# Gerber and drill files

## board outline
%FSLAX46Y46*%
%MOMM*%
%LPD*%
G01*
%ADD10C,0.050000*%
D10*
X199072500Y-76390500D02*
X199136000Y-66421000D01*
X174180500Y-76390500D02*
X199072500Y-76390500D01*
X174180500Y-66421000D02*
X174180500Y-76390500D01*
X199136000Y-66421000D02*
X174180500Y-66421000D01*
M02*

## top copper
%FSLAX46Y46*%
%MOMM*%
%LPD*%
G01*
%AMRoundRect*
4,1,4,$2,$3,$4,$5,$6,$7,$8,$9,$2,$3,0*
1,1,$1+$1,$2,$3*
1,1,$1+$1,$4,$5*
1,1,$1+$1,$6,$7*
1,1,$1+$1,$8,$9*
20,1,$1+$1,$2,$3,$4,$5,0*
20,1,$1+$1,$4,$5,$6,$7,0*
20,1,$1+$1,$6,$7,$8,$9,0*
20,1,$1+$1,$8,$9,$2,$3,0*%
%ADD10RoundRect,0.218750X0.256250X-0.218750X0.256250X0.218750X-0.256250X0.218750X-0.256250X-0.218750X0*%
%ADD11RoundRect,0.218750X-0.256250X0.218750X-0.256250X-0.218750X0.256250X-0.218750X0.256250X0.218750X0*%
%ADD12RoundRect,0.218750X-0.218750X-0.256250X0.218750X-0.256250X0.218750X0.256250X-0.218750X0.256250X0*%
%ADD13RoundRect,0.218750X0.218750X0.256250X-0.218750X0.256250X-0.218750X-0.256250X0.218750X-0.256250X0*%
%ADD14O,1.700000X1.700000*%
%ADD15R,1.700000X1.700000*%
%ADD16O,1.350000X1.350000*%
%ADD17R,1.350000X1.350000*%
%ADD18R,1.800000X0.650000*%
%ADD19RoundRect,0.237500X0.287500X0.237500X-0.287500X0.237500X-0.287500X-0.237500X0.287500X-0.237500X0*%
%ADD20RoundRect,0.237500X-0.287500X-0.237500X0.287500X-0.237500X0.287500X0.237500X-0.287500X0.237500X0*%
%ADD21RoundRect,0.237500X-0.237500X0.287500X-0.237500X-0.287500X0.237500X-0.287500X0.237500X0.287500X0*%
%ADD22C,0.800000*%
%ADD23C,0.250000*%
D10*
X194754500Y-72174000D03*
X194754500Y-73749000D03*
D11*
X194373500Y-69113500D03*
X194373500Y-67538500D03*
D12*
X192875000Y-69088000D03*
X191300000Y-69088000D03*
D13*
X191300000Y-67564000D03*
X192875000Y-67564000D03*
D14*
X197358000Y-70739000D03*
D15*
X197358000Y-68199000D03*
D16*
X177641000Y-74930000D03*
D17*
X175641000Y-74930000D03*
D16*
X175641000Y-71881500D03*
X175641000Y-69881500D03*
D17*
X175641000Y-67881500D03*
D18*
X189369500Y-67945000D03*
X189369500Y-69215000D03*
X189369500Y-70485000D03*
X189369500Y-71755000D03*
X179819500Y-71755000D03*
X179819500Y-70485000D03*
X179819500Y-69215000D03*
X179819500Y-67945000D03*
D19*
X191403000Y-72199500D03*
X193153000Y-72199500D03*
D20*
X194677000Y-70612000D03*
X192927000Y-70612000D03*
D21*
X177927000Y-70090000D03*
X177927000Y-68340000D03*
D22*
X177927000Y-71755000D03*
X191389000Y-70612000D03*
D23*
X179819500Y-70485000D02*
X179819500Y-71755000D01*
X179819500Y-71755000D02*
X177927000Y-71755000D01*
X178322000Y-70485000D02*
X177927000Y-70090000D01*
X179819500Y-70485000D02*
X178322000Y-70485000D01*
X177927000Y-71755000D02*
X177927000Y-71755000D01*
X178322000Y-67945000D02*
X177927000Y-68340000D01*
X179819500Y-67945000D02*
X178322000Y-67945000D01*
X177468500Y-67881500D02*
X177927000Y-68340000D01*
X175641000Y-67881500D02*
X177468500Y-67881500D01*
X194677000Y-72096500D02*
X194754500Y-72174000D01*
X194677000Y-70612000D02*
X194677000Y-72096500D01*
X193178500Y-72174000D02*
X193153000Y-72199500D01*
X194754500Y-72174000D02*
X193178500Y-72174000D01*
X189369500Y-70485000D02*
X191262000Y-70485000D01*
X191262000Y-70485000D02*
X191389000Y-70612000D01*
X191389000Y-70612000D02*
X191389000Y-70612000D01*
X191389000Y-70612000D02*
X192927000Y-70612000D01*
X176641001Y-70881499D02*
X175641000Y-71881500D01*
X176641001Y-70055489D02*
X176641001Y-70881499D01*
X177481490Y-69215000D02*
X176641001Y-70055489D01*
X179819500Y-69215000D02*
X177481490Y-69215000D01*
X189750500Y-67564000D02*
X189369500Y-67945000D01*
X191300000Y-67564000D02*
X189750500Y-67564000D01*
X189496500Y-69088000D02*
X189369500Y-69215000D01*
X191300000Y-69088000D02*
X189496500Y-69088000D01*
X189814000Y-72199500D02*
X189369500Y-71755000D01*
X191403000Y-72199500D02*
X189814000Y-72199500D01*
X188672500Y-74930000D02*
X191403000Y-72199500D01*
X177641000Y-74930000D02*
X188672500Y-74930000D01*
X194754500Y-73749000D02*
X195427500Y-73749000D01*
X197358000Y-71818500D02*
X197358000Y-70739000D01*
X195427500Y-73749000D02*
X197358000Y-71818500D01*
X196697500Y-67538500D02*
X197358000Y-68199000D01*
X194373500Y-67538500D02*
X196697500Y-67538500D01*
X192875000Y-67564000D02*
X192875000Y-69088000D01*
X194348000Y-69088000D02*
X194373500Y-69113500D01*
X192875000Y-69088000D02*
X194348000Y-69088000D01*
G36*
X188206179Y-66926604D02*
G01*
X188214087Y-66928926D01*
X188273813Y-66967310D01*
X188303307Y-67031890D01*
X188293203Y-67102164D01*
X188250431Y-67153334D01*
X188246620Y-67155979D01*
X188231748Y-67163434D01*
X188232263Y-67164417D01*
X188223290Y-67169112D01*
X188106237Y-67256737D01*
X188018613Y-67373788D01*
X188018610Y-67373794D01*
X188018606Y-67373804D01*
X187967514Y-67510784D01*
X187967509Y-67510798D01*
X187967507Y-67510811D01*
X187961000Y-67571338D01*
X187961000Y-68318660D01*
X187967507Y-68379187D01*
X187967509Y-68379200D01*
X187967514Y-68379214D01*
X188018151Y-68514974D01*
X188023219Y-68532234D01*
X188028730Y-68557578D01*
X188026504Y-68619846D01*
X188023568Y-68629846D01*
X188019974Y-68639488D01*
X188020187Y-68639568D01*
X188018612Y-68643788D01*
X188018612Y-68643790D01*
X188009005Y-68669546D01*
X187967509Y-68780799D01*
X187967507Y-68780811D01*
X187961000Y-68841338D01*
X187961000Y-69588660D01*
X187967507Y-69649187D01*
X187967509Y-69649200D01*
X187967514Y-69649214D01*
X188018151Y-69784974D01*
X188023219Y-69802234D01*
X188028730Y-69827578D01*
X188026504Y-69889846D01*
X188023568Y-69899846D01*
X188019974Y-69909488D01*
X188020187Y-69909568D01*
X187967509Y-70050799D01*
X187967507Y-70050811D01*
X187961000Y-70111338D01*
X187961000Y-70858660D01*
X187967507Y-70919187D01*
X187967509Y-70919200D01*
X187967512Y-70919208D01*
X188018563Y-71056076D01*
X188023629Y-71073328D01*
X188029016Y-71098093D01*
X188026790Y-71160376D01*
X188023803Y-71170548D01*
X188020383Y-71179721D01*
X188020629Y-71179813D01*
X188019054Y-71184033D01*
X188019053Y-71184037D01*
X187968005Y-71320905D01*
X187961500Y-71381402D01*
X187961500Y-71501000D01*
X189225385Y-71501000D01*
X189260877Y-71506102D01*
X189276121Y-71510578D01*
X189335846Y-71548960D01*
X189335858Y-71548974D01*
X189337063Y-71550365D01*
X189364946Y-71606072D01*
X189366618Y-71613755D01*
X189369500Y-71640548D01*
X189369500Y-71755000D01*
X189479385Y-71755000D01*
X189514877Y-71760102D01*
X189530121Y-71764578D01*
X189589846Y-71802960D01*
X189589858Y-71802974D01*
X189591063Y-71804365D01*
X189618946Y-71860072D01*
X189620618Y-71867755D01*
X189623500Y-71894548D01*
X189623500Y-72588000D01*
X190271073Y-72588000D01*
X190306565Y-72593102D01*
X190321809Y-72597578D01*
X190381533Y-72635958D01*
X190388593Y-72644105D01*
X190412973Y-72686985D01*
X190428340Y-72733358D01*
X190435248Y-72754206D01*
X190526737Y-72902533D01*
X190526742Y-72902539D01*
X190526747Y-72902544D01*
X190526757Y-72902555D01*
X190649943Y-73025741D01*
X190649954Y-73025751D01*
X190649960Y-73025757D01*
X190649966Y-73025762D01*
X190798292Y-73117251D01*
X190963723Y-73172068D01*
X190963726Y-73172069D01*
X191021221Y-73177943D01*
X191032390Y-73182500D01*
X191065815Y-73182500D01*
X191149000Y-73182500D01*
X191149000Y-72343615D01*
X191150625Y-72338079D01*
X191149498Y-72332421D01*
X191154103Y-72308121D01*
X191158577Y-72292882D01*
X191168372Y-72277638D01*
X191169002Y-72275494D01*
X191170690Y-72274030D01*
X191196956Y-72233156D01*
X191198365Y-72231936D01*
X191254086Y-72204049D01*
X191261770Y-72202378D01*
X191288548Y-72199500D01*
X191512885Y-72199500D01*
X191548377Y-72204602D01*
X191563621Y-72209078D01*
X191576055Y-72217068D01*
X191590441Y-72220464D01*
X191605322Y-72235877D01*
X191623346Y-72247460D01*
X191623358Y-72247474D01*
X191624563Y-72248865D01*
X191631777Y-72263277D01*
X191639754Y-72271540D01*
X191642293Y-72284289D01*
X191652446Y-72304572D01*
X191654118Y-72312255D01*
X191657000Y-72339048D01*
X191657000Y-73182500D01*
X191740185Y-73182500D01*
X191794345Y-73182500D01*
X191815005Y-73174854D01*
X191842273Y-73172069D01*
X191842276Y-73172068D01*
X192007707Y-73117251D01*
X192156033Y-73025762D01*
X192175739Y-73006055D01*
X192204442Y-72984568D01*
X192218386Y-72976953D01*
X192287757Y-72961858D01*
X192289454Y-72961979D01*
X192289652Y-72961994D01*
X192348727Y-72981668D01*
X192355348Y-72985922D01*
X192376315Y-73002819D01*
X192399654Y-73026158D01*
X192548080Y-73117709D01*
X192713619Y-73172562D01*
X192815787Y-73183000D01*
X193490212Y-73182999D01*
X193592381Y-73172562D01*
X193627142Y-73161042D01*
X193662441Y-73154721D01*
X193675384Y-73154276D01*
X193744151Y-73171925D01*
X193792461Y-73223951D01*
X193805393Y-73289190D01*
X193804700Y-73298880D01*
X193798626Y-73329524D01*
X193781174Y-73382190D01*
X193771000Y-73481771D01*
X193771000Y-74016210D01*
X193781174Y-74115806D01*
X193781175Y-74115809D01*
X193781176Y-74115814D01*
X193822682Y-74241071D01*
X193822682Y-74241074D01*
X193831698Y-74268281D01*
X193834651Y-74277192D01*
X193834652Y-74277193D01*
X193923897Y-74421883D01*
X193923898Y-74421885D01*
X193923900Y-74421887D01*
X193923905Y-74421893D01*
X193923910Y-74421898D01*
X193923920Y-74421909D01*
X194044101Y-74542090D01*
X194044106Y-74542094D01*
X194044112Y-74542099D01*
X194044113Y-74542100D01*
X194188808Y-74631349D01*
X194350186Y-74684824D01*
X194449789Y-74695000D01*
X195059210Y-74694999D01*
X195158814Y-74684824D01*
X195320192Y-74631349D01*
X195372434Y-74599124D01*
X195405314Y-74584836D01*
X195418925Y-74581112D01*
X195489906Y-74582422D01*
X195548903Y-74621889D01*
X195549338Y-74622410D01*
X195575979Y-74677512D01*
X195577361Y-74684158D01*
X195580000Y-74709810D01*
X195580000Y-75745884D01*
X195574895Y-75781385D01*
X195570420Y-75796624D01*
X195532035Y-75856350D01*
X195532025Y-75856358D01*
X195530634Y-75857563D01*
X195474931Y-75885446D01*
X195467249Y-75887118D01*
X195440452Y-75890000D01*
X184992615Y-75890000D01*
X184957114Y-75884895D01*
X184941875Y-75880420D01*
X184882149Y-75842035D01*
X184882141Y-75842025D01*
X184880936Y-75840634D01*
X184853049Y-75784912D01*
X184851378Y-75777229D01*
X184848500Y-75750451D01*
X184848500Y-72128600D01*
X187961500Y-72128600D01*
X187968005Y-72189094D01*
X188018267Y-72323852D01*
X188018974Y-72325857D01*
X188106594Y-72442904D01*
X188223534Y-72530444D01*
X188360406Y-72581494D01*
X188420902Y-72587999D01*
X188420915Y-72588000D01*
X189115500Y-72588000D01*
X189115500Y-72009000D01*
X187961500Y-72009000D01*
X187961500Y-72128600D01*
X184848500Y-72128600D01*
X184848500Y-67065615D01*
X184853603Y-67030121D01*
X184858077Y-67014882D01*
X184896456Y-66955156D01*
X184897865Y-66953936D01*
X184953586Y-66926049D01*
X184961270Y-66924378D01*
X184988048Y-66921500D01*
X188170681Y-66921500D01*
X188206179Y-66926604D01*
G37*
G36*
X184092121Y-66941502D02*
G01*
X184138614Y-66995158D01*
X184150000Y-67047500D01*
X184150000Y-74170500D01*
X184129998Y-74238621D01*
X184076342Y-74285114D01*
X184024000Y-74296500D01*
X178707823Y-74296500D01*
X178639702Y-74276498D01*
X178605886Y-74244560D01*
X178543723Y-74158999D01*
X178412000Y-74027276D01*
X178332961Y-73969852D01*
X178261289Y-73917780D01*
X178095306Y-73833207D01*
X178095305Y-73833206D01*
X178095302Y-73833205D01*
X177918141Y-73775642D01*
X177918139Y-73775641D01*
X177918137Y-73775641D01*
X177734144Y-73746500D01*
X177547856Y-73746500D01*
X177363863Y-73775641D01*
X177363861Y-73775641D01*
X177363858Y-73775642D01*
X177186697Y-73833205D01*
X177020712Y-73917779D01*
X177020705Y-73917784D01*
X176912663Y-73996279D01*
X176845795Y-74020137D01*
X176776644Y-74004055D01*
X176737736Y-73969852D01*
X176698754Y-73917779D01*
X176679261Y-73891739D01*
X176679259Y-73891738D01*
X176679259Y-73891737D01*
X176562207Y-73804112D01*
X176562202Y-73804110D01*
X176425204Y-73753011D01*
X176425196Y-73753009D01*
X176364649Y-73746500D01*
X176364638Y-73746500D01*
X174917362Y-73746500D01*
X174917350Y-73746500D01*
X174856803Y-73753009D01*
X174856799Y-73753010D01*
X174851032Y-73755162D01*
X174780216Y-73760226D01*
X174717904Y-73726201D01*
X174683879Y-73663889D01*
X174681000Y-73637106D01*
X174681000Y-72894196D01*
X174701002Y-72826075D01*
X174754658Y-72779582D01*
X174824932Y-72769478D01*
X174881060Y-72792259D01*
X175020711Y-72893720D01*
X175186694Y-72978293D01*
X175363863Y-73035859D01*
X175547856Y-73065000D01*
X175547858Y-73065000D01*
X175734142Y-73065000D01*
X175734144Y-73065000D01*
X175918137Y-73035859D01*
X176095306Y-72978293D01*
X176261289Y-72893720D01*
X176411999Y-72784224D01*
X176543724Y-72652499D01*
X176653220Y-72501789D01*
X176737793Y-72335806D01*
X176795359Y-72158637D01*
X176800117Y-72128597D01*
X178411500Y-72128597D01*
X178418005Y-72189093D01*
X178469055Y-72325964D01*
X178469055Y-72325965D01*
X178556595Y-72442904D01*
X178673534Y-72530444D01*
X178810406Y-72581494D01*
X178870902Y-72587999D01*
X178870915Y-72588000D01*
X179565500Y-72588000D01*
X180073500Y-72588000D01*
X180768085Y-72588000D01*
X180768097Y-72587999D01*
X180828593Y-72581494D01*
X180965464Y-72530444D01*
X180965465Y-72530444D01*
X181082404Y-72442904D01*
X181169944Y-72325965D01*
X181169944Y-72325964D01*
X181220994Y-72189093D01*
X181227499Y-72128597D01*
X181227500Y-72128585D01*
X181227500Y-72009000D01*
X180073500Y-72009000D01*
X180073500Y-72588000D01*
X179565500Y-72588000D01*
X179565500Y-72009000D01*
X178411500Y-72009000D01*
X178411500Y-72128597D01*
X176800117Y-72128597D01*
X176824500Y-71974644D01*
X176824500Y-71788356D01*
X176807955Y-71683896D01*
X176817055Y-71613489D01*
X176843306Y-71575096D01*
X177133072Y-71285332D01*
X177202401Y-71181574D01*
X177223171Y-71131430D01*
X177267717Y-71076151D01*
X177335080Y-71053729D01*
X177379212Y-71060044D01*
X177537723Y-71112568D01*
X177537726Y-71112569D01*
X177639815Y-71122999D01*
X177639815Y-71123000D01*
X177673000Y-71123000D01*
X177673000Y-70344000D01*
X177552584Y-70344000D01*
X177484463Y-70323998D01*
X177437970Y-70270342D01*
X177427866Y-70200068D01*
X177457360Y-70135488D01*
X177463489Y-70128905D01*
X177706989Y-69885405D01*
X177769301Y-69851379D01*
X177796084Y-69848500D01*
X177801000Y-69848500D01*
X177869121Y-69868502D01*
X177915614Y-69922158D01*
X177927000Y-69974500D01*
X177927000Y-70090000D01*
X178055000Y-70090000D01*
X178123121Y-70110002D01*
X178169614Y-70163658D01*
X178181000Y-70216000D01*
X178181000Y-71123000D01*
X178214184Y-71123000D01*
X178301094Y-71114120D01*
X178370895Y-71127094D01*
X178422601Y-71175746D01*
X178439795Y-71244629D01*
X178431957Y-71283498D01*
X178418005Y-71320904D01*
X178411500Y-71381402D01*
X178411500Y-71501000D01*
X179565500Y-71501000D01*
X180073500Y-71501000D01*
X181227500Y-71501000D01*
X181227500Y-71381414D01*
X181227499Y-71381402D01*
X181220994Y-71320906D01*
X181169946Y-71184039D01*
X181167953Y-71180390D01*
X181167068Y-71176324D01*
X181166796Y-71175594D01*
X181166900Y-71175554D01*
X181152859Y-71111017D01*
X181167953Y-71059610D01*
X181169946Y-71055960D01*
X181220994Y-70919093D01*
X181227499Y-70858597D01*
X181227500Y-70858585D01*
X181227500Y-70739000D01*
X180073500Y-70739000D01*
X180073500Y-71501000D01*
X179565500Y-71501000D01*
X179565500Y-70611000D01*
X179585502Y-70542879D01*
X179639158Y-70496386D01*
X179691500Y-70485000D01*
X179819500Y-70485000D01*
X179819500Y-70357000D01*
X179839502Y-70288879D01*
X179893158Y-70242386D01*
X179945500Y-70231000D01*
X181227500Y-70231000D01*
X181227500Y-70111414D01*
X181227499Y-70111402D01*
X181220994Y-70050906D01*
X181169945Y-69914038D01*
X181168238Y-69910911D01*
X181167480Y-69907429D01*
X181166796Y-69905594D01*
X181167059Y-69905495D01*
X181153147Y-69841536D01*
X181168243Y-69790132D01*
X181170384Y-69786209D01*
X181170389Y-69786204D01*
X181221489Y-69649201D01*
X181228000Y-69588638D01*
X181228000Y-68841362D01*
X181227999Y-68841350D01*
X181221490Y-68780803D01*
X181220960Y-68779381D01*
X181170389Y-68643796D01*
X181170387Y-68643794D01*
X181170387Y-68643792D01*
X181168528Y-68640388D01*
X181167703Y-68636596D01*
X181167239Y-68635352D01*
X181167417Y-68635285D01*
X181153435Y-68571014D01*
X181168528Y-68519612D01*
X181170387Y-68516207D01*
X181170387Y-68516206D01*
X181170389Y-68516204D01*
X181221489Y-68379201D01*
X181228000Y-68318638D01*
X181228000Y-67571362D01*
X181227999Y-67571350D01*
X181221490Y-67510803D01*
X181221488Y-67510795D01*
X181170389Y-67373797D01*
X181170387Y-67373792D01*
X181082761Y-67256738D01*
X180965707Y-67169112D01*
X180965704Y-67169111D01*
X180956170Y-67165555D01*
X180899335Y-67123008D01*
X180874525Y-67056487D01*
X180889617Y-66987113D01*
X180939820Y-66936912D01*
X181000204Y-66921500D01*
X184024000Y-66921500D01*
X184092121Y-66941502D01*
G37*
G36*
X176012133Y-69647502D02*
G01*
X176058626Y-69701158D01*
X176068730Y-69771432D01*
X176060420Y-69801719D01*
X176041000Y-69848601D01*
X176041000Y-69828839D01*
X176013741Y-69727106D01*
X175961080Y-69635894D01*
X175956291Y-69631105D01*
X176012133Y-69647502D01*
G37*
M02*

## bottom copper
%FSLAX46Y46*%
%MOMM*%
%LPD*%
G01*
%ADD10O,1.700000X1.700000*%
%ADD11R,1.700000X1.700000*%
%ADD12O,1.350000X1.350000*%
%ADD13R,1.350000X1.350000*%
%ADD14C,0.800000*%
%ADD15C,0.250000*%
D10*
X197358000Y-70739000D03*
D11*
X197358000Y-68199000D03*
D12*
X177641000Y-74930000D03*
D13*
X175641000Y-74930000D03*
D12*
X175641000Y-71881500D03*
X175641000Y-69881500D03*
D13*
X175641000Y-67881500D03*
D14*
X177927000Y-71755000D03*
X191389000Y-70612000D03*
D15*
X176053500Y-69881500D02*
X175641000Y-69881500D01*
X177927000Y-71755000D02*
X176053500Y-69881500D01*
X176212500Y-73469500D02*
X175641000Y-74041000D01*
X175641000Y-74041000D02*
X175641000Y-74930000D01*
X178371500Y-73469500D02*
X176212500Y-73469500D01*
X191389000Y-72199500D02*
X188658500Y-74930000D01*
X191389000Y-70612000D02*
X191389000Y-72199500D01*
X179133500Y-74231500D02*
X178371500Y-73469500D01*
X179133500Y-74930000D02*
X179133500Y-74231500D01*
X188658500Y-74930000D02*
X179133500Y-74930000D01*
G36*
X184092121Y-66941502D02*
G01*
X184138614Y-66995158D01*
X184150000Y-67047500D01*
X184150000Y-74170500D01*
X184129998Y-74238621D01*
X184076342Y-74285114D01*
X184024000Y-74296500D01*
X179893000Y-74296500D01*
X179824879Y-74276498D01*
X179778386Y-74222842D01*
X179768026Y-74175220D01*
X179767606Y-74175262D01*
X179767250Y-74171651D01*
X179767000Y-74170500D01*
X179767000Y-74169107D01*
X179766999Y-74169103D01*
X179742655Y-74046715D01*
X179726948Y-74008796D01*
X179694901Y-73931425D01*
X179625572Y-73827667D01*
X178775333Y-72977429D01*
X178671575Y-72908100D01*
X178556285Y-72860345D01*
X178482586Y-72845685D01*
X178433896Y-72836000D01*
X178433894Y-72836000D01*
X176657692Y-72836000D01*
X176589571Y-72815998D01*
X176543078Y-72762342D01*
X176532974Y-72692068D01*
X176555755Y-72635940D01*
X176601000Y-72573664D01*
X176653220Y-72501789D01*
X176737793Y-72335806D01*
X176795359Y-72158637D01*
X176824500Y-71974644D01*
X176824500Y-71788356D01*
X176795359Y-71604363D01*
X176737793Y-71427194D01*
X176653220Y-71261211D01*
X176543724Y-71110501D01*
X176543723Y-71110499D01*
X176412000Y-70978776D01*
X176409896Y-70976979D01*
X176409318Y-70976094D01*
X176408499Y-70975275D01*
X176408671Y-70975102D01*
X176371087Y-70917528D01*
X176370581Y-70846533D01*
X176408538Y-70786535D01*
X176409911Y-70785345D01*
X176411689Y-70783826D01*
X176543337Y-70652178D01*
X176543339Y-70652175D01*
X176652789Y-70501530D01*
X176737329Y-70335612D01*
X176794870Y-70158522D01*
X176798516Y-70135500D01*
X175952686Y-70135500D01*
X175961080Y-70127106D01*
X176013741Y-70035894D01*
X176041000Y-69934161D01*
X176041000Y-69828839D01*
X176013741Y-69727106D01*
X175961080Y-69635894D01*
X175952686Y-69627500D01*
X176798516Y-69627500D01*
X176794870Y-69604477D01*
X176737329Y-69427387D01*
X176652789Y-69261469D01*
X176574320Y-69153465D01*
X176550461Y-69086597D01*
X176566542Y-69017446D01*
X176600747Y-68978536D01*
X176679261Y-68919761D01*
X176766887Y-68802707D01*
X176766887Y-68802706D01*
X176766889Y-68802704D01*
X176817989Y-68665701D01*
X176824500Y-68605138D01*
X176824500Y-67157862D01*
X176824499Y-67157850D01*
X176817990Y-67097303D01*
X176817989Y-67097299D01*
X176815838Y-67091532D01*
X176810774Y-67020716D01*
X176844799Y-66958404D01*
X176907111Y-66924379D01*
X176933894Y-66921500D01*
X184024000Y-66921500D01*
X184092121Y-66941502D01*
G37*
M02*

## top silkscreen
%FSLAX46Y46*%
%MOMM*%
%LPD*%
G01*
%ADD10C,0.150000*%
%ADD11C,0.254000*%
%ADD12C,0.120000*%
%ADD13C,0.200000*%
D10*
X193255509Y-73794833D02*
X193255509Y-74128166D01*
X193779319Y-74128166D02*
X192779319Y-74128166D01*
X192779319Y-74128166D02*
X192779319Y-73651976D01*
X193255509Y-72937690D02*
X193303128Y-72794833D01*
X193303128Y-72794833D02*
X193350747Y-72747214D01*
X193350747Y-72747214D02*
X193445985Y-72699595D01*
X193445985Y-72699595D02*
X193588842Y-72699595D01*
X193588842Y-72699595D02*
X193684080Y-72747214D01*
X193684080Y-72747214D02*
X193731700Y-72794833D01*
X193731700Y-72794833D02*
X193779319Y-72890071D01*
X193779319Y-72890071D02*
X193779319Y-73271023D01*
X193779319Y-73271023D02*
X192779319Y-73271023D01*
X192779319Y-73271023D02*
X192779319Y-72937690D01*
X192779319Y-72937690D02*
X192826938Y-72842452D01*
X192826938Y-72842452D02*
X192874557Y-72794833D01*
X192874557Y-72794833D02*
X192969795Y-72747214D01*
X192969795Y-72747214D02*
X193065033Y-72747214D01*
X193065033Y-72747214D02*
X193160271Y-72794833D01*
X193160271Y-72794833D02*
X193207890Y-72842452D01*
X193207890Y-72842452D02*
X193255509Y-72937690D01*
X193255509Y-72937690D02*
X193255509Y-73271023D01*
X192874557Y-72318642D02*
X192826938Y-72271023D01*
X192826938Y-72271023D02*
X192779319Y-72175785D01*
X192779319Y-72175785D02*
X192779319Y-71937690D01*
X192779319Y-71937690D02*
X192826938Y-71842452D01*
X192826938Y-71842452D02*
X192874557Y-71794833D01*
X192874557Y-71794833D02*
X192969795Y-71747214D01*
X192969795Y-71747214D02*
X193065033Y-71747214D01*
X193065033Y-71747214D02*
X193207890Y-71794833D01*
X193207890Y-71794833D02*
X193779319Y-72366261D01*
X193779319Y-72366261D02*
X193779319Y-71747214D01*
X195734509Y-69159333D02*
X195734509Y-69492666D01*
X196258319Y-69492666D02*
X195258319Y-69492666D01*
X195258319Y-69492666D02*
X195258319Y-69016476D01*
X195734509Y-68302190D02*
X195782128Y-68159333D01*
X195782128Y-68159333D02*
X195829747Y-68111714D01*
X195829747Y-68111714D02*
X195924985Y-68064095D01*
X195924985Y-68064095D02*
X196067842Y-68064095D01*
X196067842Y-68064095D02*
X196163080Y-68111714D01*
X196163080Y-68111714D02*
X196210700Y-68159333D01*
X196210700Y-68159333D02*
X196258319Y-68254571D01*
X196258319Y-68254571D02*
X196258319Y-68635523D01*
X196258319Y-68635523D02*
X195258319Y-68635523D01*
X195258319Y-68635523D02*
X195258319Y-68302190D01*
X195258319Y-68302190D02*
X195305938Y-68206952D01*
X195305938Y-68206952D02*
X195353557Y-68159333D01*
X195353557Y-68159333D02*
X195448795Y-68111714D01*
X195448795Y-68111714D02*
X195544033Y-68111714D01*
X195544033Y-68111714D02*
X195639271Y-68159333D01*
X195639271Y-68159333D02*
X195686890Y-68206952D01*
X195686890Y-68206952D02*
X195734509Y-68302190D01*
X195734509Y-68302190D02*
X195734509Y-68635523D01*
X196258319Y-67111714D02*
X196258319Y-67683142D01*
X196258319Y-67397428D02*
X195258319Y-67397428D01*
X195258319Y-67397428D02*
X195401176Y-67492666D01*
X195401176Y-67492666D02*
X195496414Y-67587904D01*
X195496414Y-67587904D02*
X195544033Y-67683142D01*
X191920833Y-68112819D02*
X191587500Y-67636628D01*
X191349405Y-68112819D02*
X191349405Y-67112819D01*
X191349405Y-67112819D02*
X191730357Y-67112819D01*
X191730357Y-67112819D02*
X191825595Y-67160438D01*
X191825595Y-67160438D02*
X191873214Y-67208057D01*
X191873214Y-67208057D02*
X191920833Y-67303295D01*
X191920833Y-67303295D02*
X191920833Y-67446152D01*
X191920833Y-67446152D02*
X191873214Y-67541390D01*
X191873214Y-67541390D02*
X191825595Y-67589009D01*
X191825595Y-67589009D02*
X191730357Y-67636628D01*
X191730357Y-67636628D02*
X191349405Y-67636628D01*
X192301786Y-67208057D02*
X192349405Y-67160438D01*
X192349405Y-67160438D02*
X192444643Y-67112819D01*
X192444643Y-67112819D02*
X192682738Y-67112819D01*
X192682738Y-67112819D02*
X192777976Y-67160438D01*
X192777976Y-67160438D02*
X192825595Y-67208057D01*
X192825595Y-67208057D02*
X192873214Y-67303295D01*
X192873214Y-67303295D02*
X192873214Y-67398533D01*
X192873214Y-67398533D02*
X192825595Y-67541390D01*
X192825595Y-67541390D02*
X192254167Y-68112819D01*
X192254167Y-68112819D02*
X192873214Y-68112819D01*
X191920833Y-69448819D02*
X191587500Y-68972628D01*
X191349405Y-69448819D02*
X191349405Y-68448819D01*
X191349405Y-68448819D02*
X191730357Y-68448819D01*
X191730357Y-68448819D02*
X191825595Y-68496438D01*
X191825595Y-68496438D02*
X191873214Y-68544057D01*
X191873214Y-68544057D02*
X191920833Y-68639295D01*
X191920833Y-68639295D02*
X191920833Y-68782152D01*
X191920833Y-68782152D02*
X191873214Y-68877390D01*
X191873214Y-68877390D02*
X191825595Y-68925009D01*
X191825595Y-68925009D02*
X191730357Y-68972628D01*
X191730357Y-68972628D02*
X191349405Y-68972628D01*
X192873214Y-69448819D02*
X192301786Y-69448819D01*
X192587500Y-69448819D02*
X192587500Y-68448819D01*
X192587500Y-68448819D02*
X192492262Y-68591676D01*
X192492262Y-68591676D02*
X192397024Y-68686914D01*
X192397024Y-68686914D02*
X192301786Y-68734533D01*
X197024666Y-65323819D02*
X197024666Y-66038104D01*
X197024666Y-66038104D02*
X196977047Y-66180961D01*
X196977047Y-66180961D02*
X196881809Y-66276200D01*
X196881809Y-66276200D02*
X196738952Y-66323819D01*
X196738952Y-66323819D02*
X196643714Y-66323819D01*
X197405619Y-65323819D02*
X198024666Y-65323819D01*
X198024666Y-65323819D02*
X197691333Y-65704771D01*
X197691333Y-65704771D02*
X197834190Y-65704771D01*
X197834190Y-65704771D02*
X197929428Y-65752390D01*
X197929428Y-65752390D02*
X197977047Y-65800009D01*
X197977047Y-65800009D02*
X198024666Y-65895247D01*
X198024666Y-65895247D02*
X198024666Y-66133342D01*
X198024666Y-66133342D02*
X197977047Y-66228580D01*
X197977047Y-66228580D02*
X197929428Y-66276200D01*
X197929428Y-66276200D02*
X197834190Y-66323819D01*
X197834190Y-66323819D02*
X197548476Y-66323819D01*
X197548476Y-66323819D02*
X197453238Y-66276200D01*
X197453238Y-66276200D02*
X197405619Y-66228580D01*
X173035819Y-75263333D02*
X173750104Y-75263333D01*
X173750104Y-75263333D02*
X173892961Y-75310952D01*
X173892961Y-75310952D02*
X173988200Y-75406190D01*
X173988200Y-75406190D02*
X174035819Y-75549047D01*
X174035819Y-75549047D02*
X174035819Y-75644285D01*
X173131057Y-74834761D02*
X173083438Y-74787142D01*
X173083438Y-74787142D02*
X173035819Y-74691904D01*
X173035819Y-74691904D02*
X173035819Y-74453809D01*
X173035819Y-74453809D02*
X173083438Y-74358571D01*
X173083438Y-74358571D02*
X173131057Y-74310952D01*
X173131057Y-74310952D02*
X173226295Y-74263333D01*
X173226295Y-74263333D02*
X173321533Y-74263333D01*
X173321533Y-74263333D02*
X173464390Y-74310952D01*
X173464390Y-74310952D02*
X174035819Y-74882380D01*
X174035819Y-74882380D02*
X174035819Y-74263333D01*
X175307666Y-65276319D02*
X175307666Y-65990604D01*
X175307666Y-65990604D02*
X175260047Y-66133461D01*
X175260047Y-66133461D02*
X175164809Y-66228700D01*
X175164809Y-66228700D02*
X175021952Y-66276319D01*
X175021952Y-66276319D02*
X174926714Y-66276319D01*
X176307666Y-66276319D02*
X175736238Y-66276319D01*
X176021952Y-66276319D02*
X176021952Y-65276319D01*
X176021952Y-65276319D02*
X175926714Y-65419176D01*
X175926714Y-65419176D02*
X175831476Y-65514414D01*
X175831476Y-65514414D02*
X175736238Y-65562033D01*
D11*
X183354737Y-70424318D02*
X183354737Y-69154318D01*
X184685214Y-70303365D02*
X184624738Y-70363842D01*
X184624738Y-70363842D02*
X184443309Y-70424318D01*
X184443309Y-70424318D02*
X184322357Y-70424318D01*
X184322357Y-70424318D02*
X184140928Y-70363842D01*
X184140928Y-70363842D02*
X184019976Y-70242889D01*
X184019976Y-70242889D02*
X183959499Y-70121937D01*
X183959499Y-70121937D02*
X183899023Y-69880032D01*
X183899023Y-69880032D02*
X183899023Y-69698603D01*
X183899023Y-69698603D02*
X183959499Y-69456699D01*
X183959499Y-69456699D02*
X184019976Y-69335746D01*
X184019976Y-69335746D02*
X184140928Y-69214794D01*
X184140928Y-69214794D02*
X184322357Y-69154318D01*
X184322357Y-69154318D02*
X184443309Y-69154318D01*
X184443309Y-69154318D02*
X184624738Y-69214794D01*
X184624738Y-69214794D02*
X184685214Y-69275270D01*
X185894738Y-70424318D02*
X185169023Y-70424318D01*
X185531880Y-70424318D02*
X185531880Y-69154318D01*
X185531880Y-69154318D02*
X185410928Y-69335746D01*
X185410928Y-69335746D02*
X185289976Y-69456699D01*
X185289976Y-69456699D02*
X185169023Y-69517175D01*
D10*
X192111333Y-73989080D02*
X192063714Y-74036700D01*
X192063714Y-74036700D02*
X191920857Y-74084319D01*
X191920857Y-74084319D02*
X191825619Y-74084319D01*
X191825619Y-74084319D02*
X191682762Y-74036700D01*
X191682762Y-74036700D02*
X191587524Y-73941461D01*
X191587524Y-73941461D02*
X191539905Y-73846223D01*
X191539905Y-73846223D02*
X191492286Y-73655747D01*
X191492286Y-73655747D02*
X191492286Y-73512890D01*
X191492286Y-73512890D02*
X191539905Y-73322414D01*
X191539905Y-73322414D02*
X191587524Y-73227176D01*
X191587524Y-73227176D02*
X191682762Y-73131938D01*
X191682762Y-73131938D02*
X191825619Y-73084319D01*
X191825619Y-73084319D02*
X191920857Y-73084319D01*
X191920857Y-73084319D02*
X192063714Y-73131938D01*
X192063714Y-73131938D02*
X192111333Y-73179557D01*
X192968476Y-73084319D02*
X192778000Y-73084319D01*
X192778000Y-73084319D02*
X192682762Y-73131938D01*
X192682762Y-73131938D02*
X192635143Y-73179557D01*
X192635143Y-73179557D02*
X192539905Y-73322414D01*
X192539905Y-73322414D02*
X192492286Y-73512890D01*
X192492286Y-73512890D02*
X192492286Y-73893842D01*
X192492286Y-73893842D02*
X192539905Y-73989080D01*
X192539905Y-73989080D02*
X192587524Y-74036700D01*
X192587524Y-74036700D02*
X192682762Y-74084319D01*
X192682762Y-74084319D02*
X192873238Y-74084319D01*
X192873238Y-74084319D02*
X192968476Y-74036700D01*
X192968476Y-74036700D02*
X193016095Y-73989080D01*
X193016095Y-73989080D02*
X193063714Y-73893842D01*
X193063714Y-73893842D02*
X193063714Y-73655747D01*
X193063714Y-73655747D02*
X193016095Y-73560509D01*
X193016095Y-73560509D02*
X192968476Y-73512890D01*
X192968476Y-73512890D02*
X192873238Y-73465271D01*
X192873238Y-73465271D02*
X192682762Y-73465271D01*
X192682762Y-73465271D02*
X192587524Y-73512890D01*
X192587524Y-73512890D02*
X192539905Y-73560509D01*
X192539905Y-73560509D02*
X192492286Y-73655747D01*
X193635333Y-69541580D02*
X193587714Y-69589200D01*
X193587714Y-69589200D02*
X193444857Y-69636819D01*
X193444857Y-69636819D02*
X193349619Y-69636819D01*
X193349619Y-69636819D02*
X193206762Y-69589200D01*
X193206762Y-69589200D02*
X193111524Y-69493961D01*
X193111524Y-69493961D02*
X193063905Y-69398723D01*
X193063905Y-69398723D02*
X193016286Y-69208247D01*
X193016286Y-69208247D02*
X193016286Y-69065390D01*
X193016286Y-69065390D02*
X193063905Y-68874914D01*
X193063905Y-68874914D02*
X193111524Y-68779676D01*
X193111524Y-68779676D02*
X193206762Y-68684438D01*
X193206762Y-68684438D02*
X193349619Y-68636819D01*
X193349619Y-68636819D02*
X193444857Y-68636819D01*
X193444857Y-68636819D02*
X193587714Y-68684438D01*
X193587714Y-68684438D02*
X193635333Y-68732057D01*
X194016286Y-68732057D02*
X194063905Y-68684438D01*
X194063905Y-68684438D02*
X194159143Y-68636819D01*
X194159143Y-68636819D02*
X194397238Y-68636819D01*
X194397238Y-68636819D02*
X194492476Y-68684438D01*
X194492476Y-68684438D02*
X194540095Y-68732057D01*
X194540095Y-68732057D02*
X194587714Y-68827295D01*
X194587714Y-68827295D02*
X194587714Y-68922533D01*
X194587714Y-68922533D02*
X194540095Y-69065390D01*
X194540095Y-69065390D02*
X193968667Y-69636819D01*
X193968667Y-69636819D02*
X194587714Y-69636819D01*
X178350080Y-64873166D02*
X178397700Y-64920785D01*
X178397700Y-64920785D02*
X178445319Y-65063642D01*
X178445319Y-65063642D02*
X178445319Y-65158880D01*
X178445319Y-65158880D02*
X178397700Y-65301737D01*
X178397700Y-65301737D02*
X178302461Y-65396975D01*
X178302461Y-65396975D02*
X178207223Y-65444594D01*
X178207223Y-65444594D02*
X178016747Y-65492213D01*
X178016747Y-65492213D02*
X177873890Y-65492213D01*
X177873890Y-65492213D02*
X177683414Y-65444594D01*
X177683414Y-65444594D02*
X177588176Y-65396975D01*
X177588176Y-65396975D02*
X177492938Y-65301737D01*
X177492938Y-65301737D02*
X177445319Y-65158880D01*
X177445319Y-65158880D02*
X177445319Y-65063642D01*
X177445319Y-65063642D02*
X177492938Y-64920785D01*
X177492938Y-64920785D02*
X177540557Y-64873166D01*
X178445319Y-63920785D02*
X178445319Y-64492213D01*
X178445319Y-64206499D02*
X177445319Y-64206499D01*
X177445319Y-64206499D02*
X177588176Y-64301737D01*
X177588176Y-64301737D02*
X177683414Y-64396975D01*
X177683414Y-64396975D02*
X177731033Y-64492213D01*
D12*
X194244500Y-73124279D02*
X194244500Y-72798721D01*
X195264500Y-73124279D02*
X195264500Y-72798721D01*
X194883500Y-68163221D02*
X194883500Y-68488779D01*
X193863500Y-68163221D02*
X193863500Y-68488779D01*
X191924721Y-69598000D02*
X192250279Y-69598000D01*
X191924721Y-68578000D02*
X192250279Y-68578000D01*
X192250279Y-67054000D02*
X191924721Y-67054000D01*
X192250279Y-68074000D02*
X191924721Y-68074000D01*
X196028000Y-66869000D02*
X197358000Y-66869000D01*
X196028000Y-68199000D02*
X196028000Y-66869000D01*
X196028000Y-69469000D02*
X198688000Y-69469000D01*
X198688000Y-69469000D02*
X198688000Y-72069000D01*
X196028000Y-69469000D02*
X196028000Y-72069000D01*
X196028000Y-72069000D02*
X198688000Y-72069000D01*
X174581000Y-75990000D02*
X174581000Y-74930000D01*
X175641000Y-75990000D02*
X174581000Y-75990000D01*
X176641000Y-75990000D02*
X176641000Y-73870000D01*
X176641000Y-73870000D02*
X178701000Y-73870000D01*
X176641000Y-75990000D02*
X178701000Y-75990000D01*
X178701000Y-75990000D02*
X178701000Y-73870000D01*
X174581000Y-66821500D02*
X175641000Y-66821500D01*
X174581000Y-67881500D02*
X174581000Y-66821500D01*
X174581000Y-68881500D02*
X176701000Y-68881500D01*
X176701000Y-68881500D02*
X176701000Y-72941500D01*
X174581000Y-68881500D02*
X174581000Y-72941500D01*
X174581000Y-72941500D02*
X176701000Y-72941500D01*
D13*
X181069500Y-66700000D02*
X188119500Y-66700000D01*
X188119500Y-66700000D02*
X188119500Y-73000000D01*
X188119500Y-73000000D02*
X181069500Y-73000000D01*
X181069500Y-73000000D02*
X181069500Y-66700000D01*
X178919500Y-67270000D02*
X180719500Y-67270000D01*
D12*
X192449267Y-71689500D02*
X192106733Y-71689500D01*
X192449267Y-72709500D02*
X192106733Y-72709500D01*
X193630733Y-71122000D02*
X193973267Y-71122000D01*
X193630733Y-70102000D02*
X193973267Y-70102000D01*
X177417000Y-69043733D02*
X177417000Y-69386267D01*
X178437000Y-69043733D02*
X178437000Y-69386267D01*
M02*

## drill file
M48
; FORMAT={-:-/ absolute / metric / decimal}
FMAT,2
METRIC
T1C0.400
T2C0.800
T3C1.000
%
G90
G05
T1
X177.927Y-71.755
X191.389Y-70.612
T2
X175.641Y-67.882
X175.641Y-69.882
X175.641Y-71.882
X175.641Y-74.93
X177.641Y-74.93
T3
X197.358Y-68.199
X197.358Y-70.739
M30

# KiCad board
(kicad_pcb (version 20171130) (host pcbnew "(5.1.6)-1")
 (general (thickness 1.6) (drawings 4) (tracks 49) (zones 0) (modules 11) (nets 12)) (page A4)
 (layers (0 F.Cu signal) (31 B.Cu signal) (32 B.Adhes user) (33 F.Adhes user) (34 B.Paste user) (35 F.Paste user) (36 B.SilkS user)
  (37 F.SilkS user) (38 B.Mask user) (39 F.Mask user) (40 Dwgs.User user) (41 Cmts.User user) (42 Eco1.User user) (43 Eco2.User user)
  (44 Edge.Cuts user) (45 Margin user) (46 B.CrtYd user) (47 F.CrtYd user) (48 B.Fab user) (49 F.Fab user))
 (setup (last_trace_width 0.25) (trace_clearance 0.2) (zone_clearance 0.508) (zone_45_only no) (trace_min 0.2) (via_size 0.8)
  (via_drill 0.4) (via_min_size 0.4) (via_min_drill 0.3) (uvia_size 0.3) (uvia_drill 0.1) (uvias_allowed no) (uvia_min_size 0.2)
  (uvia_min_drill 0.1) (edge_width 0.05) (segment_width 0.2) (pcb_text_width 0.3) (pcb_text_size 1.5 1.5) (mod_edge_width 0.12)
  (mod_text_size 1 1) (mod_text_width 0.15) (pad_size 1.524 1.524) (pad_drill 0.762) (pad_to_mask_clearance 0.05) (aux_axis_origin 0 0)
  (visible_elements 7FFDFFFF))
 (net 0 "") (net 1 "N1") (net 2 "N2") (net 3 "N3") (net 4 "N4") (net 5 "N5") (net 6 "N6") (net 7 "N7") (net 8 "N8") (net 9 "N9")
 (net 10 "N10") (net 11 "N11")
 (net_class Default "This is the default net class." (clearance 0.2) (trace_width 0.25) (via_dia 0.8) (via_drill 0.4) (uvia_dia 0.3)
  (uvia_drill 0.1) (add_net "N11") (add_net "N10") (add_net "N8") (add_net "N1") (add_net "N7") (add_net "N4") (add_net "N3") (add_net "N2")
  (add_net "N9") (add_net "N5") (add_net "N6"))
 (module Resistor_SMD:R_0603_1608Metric (layer F.Cu) (at 194.7545 72.9615 90)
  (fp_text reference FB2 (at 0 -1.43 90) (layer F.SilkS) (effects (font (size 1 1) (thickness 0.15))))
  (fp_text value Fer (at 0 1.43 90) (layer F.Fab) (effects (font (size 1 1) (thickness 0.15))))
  (fp_line (start -0.162779 -0.51) (end 0.162779 -0.51) (layer F.SilkS) (width 0.12))
  (fp_line (start -0.162779 0.51) (end 0.162779 0.51) (layer F.SilkS) (width 0.12))
  (pad 2 smd roundrect (at 0.7875 0 90) (size 0.875 0.95) (layers F.Cu F.Paste F.Mask) (roundrect_rratio 0.25) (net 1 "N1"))
  (pad 1 smd roundrect (at -0.7875 0 90) (size 0.875 0.95) (layers F.Cu F.Paste F.Mask) (roundrect_rratio 0.25) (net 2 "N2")))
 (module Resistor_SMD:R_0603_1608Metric (layer F.Cu) (at 194.3735 68.326 270)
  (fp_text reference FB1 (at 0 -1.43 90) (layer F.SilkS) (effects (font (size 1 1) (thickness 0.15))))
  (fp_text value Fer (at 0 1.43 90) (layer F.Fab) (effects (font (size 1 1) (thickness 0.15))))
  (fp_line (start -0.162779 -0.51) (end 0.162779 -0.51) (layer F.SilkS) (width 0.12))
  (fp_line (start -0.162779 0.51) (end 0.162779 0.51) (layer F.SilkS) (width 0.12))
  (pad 2 smd roundrect (at 0.7875 0 270) (size 0.875 0.95) (layers F.Cu F.Paste F.Mask) (roundrect_rratio 0.25) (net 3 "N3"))
  (pad 1 smd roundrect (at -0.7875 0 270) (size 0.875 0.95) (layers F.Cu F.Paste F.Mask) (roundrect_rratio 0.25) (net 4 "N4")))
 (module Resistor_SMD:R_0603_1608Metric (layer F.Cu) (at 192.0875 69.088)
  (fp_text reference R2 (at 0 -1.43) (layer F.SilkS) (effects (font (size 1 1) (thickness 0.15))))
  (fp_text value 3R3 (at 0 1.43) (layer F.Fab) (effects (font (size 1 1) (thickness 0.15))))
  (fp_line (start -0.162779 0.51) (end 0.162779 0.51) (layer F.SilkS) (width 0.12))
  (fp_line (start -0.162779 -0.51) (end 0.162779 -0.51) (layer F.SilkS) (width 0.12))
  (pad 2 smd roundrect (at 0.7875 0) (size 0.875 0.95) (layers F.Cu F.Paste F.Mask) (roundrect_rratio 0.25) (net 3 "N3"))
  (pad 1 smd roundrect (at -0.7875 0) (size 0.875 0.95) (layers F.Cu F.Paste F.Mask) (roundrect_rratio 0.25) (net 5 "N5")))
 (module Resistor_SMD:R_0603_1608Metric (layer F.Cu) (at 192.0875 67.564 180)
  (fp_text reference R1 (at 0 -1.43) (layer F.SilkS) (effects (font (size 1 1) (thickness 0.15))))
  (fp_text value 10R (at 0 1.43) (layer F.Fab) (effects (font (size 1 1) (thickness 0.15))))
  (fp_line (start -0.162779 0.51) (end 0.162779 0.51) (layer F.SilkS) (width 0.12))
  (fp_line (start -0.162779 -0.51) (end 0.162779 -0.51) (layer F.SilkS) (width 0.12))
  (pad 2 smd roundrect (at 0.7875 0 180) (size 0.875 0.95) (layers F.Cu F.Paste F.Mask) (roundrect_rratio 0.25) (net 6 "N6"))
  (pad 1 smd roundrect (at -0.7875 0 180) (size 0.875 0.95) (layers F.Cu F.Paste F.Mask) (roundrect_rratio 0.25) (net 3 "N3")))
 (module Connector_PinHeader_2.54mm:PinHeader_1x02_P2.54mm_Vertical (layer F.Cu) (at 197.358 68.199)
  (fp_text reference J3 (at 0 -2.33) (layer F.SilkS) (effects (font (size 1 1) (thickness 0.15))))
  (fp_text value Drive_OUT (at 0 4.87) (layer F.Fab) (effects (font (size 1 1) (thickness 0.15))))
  (fp_line (start -1.33 -1.33) (end 0 -1.33) (layer F.SilkS) (width 0.12))
  (fp_line (start -1.33 0) (end -1.33 -1.33) (layer F.SilkS) (width 0.12))
  (fp_line (start -1.33 1.27) (end 1.33 1.27) (layer F.SilkS) (width 0.12))
  (fp_line (start 1.33 1.27) (end 1.33 3.87) (layer F.SilkS) (width 0.12))
  (fp_line (start -1.33 1.27) (end -1.33 3.87) (layer F.SilkS) (width 0.12))
  (fp_line (start -1.33 3.87) (end 1.33 3.87) (layer F.SilkS) (width 0.12))
  (pad 2 thru_hole oval (at 0 2.54) (size 1.7 1.7) (drill 1) (layers *.Cu *.Mask) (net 2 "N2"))
  (pad 1 thru_hole rect (at 0 0) (size 1.7 1.7) (drill 1) (layers *.Cu *.Mask) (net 4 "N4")))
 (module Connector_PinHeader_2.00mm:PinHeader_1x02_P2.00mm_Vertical (layer F.Cu) (at 175.641 74.93 90)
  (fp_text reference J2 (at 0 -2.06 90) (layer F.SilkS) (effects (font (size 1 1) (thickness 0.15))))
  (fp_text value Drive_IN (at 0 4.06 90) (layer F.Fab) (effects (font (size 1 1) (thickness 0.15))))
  (fp_line (start -1.06 -1.06) (end 0 -1.06) (layer F.SilkS) (width 0.12))
  (fp_line (start -1.06 0) (end -1.06 -1.06) (layer F.SilkS) (width 0.12))
  (fp_line (start -1.06 1) (end 1.06 1) (layer F.SilkS) (width 0.12))
  (fp_line (start 1.06 1) (end 1.06 3.06) (layer F.SilkS) (width 0.12))
  (fp_line (start -1.06 1) (end -1.06 3.06) (layer F.SilkS) (width 0.12))
  (fp_line (start -1.06 3.06) (end 1.06 3.06) (layer F.SilkS) (width 0.12))
  (pad 2 thru_hole oval (at 0 2 90) (size 1.35 1.35) (drill 0.8) (layers *.Cu *.Mask) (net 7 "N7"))
  (pad 1 thru_hole rect (at 0 0 90) (size 1.35 1.35) (drill 0.8) (layers *.Cu *.Mask) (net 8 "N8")))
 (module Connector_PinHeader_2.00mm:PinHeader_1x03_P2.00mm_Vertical (layer F.Cu) (at 175.641 67.8815)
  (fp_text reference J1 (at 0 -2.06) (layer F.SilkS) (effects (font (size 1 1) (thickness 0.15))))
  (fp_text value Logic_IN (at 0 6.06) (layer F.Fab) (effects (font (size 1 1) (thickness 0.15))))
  (fp_line (start -1.06 -1.06) (end 0 -1.06) (layer F.SilkS) (width 0.12))
  (fp_line (start -1.06 0) (end -1.06 -1.06) (layer F.SilkS) (width 0.12))
  (fp_line (start -1.06 1) (end 1.06 1) (layer F.SilkS) (width 0.12))
  (fp_line (start 1.06 1) (end 1.06 5.06) (layer F.SilkS) (width 0.12))
  (fp_line (start -1.06 1) (end -1.06 5.06) (layer F.SilkS) (width 0.12))
  (fp_line (start -1.06 5.06) (end 1.06 5.06) (layer F.SilkS) (width 0.12))
  (pad 3 thru_hole oval (at 0 4) (size 1.35 1.35) (drill 0.8) (layers *.Cu *.Mask) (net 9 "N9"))
  (pad 2 thru_hole oval (at 0 2) (size 1.35 1.35) (drill 0.8) (layers *.Cu *.Mask) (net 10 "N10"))
  (pad 1 thru_hole rect (at 0 0) (size 1.35 1.35) (drill 0.8) (layers *.Cu *.Mask) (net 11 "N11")))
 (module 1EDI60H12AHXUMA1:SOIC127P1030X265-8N (layer F.Cu) (at 184.5945 69.85)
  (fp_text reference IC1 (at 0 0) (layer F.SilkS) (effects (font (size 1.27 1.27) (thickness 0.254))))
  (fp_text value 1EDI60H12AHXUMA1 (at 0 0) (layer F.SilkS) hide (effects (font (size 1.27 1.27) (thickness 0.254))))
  (fp_line (start -3.525 -3.15) (end 3.525 -3.15) (layer F.SilkS) (width 0.2))
  (fp_line (start 3.525 -3.15) (end 3.525 3.15) (layer F.SilkS) (width 0.2))
  (fp_line (start 3.525 3.15) (end -3.525 3.15) (layer F.SilkS) (width 0.2))
  (fp_line (start -3.525 3.15) (end -3.525 -3.15) (layer F.SilkS) (width 0.2))
  (fp_line (start -5.675 -2.58) (end -3.875 -2.58) (layer F.SilkS) (width 0.2))
  (pad 8 smd rect (at 4.775 -1.905 90) (size 0.65 1.8) (layers F.Cu F.Paste F.Mask) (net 6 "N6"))
  (pad 7 smd rect (at 4.775 -0.635 90) (size 0.65 1.8) (layers F.Cu F.Paste F.Mask) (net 5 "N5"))
  (pad 6 smd rect (at 4.775 0.635 90) (size 0.65 1.8) (layers F.Cu F.Paste F.Mask) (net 8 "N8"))
  (pad 5 smd rect (at 4.775 1.905 90) (size 0.65 1.8) (layers F.Cu F.Paste F.Mask) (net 7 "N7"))
  (pad 4 smd rect (at -4.775 1.905 90) (size 0.65 1.8) (layers F.Cu F.Paste F.Mask) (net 10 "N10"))
  (pad 3 smd rect (at -4.775 0.635 90) (size 0.65 1.8) (layers F.Cu F.Paste F.Mask) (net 10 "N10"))
  (pad 2 smd rect (at -4.775 -0.635 90) (size 0.65 1.8) (layers F.Cu F.Paste F.Mask) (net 9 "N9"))
  (pad 1 smd rect (at -4.775 -1.905 90) (size 0.65 1.8) (layers F.Cu F.Paste F.Mask) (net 11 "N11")))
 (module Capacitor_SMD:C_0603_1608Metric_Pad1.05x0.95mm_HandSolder (layer F.Cu) (at 192.278 72.1995 180)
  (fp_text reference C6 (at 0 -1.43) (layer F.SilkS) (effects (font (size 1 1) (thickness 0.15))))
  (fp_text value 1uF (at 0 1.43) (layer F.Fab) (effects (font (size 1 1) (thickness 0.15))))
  (fp_line (start -0.171267 0.51) (end 0.171267 0.51) (layer F.SilkS) (width 0.12))
  (fp_line (start -0.171267 -0.51) (end 0.171267 -0.51) (layer F.SilkS) (width 0.12))
  (pad 2 smd roundrect (at 0.875 0 180) (size 1.05 0.95) (layers F.Cu F.Paste F.Mask) (roundrect_rratio 0.25) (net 7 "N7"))
  (pad 1 smd roundrect (at -0.875 0 180) (size 1.05 0.95) (layers F.Cu F.Paste F.Mask) (roundrect_rratio 0.25) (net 1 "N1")))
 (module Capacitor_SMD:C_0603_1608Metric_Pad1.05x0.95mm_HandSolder (layer F.Cu) (at 193.802 70.612)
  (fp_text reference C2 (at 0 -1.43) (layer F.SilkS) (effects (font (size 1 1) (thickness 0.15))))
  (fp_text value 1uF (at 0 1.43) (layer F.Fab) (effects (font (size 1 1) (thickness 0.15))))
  (fp_line (start -0.171267 0.51) (end 0.171267 0.51) (layer F.SilkS) (width 0.12))
  (fp_line (start -0.171267 -0.51) (end 0.171267 -0.51) (layer F.SilkS) (width 0.12))
  (pad 2 smd roundrect (at 0.875 0) (size 1.05 0.95) (layers F.Cu F.Paste F.Mask) (roundrect_rratio 0.25) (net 1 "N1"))
  (pad 1 smd roundrect (at -0.875 0) (size 1.05 0.95) (layers F.Cu F.Paste F.Mask) (roundrect_rratio 0.25) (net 8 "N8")))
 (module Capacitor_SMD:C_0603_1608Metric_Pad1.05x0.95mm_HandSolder (layer F.Cu) (at 177.927 69.215 270)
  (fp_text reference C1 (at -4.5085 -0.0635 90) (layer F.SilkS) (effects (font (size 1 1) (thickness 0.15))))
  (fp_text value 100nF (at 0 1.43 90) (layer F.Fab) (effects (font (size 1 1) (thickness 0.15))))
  (fp_line (start -0.171267 0.51) (end 0.171267 0.51) (layer F.SilkS) (width 0.12))
  (fp_line (start -0.171267 -0.51) (end 0.171267 -0.51) (layer F.SilkS) (width 0.12))
  (pad 2 smd roundrect (at 0.875 0 270) (size 1.05 0.95) (layers F.Cu F.Paste F.Mask) (roundrect_rratio 0.25) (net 10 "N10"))
  (pad 1 smd roundrect (at -0.875 0 270) (size 1.05 0.95) (layers F.Cu F.Paste F.Mask) (roundrect_rratio 0.25) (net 11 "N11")))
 (gr_line (start 199.0725 76.3905) (end 199.136 66.421) (layer Edge.Cuts) (width 0.05))
 (gr_line (start 174.1805 76.3905) (end 199.0725 76.3905) (layer Edge.Cuts) (width 0.05))
 (gr_line (start 174.1805 66.421) (end 174.1805 76.3905) (layer Edge.Cuts) (width 0.05))
 (gr_line (start 199.136 66.421) (end 174.1805 66.421) (layer Edge.Cuts) (width 0.05))
 (segment (start 179.8195 70.485) (end 179.8195 71.755) (width 0.25) (layer F.Cu) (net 10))
 (segment (start 179.8195 71.755) (end 177.927 71.755) (width 0.25) (layer F.Cu) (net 10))
 (segment (start 178.322 70.485) (end 177.927 70.09) (width 0.25) (layer F.Cu) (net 10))
 (segment (start 179.8195 70.485) (end 178.322 70.485) (width 0.25) (layer F.Cu) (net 10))
 (segment (start 177.927 71.755) (end 177.927 71.755) (width 0.25) (layer F.Cu) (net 10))
 (via (at 177.927 71.755) (size 0.8) (drill 0.4) (layers F.Cu B.Cu) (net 10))
 (segment (start 176.0535 69.8815) (end 175.641 69.8815) (width 0.25) (layer B.Cu) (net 10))
 (segment (start 177.927 71.755) (end 176.0535 69.8815) (width 0.25) (layer B.Cu) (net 10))
 (segment (start 178.322 67.945) (end 177.927 68.34) (width 0.25) (layer F.Cu) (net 11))
 (segment (start 179.8195 67.945) (end 178.322 67.945) (width 0.25) (layer F.Cu) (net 11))
 (segment (start 177.4685 67.8815) (end 177.927 68.34) (width 0.25) (layer F.Cu) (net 11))
 (segment (start 175.641 67.8815) (end 177.4685 67.8815) (width 0.25) (layer F.Cu) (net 11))
 (segment (start 194.677 72.0965) (end 194.7545 72.174) (width 0.25) (layer F.Cu) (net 1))
 (segment (start 194.677 70.612) (end 194.677 72.0965) (width 0.25) (layer F.Cu) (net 1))
 (segment (start 193.1785 72.174) (end 193.153 72.1995) (width 0.25) (layer F.Cu) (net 1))
 (segment (start 194.7545 72.174) (end 193.1785 72.174) (width 0.25) (layer F.Cu) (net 1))
 (segment (start 189.3695 70.485) (end 191.262 70.485) (width 0.25) (layer F.Cu) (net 8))
 (segment (start 191.262 70.485) (end 191.389 70.612) (width 0.25) (layer F.Cu) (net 8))
 (segment (start 191.389 70.612) (end 191.389 70.612) (width 0.25) (layer F.Cu) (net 8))
 (via (at 191.389 70.612) (size 0.8) (drill 0.4) (layers F.Cu B.Cu) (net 8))
 (segment (start 191.389 70.612) (end 192.927 70.612) (width 0.25) (layer F.Cu) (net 8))
 (segment (start 176.2125 73.4695) (end 175.641 74.041) (width 0.25) (layer B.Cu) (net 8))
 (segment (start 175.641 74.041) (end 175.641 74.93) (width 0.25) (layer B.Cu) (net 8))
 (segment (start 178.3715 73.4695) (end 176.2125 73.4695) (width 0.25) (layer B.Cu) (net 8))
 (segment (start 191.389 72.1995) (end 188.6585 74.93) (width 0.25) (layer B.Cu) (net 8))
 (segment (start 191.389 70.612) (end 191.389 72.1995) (width 0.25) (layer B.Cu) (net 8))
 (segment (start 179.1335 74.2315) (end 178.3715 73.4695) (width 0.25) (layer B.Cu) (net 8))
 (segment (start 179.1335 74.93) (end 179.1335 74.2315) (width 0.25) (layer B.Cu) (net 8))
 (segment (start 188.6585 74.93) (end 179.1335 74.93) (width 0.25) (layer B.Cu) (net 8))
 (segment (start 176.641001 70.881499) (end 175.641 71.8815) (width 0.25) (layer F.Cu) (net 9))
 (segment (start 176.641001 70.055489) (end 176.641001 70.881499) (width 0.25) (layer F.Cu) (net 9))
 (segment (start 177.48149 69.215) (end 176.641001 70.055489) (width 0.25) (layer F.Cu) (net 9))
 (segment (start 179.8195 69.215) (end 177.48149 69.215) (width 0.25) (layer F.Cu) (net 9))
 (segment (start 189.7505 67.564) (end 189.3695 67.945) (width 0.25) (layer F.Cu) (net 6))
 (segment (start 191.3 67.564) (end 189.7505 67.564) (width 0.25) (layer F.Cu) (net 6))
 (segment (start 189.4965 69.088) (end 189.3695 69.215) (width 0.25) (layer F.Cu) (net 5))
 (segment (start 191.3 69.088) (end 189.4965 69.088) (width 0.25) (layer F.Cu) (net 5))
 (segment (start 189.814 72.1995) (end 189.3695 71.755) (width 0.25) (layer F.Cu) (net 7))
 (segment (start 191.403 72.1995) (end 189.814 72.1995) (width 0.25) (layer F.Cu) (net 7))
 (segment (start 188.6725 74.93) (end 191.403 72.1995) (width 0.25) (layer F.Cu) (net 7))
 (segment (start 177.641 74.93) (end 188.6725 74.93) (width 0.25) (layer F.Cu) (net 7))
 (segment (start 194.7545 73.749) (end 195.4275 73.749) (width 0.25) (layer F.Cu) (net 2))
 (segment (start 197.358 71.8185) (end 197.358 70.739) (width 0.25) (layer F.Cu) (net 2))
 (segment (start 195.4275 73.749) (end 197.358 71.8185) (width 0.25) (layer F.Cu) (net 2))
 (segment (start 196.6975 67.5385) (end 197.358 68.199) (width 0.25) (layer F.Cu) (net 4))
 (segment (start 194.3735 67.5385) (end 196.6975 67.5385) (width 0.25) (layer F.Cu) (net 4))
 (segment (start 192.875 67.564) (end 192.875 69.088) (width 0.25) (layer F.Cu) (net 3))
 (segment (start 194.348 69.088) (end 194.3735 69.1135) (width 0.25) (layer F.Cu) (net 3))
 (segment (start 192.875 69.088) (end 194.348 69.088) (width 0.25) (layer F.Cu) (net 3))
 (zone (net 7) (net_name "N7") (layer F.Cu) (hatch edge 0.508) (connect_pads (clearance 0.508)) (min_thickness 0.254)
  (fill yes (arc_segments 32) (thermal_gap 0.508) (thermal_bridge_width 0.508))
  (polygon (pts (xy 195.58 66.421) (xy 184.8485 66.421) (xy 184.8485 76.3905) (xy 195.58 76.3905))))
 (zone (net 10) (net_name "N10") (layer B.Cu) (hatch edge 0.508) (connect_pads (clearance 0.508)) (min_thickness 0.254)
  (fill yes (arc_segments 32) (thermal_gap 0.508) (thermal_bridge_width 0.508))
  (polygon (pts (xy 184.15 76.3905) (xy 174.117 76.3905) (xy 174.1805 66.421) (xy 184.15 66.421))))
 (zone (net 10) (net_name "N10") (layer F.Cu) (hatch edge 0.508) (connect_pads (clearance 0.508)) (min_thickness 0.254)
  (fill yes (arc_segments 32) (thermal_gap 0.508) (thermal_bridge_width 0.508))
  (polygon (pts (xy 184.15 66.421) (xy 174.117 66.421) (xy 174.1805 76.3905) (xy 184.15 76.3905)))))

